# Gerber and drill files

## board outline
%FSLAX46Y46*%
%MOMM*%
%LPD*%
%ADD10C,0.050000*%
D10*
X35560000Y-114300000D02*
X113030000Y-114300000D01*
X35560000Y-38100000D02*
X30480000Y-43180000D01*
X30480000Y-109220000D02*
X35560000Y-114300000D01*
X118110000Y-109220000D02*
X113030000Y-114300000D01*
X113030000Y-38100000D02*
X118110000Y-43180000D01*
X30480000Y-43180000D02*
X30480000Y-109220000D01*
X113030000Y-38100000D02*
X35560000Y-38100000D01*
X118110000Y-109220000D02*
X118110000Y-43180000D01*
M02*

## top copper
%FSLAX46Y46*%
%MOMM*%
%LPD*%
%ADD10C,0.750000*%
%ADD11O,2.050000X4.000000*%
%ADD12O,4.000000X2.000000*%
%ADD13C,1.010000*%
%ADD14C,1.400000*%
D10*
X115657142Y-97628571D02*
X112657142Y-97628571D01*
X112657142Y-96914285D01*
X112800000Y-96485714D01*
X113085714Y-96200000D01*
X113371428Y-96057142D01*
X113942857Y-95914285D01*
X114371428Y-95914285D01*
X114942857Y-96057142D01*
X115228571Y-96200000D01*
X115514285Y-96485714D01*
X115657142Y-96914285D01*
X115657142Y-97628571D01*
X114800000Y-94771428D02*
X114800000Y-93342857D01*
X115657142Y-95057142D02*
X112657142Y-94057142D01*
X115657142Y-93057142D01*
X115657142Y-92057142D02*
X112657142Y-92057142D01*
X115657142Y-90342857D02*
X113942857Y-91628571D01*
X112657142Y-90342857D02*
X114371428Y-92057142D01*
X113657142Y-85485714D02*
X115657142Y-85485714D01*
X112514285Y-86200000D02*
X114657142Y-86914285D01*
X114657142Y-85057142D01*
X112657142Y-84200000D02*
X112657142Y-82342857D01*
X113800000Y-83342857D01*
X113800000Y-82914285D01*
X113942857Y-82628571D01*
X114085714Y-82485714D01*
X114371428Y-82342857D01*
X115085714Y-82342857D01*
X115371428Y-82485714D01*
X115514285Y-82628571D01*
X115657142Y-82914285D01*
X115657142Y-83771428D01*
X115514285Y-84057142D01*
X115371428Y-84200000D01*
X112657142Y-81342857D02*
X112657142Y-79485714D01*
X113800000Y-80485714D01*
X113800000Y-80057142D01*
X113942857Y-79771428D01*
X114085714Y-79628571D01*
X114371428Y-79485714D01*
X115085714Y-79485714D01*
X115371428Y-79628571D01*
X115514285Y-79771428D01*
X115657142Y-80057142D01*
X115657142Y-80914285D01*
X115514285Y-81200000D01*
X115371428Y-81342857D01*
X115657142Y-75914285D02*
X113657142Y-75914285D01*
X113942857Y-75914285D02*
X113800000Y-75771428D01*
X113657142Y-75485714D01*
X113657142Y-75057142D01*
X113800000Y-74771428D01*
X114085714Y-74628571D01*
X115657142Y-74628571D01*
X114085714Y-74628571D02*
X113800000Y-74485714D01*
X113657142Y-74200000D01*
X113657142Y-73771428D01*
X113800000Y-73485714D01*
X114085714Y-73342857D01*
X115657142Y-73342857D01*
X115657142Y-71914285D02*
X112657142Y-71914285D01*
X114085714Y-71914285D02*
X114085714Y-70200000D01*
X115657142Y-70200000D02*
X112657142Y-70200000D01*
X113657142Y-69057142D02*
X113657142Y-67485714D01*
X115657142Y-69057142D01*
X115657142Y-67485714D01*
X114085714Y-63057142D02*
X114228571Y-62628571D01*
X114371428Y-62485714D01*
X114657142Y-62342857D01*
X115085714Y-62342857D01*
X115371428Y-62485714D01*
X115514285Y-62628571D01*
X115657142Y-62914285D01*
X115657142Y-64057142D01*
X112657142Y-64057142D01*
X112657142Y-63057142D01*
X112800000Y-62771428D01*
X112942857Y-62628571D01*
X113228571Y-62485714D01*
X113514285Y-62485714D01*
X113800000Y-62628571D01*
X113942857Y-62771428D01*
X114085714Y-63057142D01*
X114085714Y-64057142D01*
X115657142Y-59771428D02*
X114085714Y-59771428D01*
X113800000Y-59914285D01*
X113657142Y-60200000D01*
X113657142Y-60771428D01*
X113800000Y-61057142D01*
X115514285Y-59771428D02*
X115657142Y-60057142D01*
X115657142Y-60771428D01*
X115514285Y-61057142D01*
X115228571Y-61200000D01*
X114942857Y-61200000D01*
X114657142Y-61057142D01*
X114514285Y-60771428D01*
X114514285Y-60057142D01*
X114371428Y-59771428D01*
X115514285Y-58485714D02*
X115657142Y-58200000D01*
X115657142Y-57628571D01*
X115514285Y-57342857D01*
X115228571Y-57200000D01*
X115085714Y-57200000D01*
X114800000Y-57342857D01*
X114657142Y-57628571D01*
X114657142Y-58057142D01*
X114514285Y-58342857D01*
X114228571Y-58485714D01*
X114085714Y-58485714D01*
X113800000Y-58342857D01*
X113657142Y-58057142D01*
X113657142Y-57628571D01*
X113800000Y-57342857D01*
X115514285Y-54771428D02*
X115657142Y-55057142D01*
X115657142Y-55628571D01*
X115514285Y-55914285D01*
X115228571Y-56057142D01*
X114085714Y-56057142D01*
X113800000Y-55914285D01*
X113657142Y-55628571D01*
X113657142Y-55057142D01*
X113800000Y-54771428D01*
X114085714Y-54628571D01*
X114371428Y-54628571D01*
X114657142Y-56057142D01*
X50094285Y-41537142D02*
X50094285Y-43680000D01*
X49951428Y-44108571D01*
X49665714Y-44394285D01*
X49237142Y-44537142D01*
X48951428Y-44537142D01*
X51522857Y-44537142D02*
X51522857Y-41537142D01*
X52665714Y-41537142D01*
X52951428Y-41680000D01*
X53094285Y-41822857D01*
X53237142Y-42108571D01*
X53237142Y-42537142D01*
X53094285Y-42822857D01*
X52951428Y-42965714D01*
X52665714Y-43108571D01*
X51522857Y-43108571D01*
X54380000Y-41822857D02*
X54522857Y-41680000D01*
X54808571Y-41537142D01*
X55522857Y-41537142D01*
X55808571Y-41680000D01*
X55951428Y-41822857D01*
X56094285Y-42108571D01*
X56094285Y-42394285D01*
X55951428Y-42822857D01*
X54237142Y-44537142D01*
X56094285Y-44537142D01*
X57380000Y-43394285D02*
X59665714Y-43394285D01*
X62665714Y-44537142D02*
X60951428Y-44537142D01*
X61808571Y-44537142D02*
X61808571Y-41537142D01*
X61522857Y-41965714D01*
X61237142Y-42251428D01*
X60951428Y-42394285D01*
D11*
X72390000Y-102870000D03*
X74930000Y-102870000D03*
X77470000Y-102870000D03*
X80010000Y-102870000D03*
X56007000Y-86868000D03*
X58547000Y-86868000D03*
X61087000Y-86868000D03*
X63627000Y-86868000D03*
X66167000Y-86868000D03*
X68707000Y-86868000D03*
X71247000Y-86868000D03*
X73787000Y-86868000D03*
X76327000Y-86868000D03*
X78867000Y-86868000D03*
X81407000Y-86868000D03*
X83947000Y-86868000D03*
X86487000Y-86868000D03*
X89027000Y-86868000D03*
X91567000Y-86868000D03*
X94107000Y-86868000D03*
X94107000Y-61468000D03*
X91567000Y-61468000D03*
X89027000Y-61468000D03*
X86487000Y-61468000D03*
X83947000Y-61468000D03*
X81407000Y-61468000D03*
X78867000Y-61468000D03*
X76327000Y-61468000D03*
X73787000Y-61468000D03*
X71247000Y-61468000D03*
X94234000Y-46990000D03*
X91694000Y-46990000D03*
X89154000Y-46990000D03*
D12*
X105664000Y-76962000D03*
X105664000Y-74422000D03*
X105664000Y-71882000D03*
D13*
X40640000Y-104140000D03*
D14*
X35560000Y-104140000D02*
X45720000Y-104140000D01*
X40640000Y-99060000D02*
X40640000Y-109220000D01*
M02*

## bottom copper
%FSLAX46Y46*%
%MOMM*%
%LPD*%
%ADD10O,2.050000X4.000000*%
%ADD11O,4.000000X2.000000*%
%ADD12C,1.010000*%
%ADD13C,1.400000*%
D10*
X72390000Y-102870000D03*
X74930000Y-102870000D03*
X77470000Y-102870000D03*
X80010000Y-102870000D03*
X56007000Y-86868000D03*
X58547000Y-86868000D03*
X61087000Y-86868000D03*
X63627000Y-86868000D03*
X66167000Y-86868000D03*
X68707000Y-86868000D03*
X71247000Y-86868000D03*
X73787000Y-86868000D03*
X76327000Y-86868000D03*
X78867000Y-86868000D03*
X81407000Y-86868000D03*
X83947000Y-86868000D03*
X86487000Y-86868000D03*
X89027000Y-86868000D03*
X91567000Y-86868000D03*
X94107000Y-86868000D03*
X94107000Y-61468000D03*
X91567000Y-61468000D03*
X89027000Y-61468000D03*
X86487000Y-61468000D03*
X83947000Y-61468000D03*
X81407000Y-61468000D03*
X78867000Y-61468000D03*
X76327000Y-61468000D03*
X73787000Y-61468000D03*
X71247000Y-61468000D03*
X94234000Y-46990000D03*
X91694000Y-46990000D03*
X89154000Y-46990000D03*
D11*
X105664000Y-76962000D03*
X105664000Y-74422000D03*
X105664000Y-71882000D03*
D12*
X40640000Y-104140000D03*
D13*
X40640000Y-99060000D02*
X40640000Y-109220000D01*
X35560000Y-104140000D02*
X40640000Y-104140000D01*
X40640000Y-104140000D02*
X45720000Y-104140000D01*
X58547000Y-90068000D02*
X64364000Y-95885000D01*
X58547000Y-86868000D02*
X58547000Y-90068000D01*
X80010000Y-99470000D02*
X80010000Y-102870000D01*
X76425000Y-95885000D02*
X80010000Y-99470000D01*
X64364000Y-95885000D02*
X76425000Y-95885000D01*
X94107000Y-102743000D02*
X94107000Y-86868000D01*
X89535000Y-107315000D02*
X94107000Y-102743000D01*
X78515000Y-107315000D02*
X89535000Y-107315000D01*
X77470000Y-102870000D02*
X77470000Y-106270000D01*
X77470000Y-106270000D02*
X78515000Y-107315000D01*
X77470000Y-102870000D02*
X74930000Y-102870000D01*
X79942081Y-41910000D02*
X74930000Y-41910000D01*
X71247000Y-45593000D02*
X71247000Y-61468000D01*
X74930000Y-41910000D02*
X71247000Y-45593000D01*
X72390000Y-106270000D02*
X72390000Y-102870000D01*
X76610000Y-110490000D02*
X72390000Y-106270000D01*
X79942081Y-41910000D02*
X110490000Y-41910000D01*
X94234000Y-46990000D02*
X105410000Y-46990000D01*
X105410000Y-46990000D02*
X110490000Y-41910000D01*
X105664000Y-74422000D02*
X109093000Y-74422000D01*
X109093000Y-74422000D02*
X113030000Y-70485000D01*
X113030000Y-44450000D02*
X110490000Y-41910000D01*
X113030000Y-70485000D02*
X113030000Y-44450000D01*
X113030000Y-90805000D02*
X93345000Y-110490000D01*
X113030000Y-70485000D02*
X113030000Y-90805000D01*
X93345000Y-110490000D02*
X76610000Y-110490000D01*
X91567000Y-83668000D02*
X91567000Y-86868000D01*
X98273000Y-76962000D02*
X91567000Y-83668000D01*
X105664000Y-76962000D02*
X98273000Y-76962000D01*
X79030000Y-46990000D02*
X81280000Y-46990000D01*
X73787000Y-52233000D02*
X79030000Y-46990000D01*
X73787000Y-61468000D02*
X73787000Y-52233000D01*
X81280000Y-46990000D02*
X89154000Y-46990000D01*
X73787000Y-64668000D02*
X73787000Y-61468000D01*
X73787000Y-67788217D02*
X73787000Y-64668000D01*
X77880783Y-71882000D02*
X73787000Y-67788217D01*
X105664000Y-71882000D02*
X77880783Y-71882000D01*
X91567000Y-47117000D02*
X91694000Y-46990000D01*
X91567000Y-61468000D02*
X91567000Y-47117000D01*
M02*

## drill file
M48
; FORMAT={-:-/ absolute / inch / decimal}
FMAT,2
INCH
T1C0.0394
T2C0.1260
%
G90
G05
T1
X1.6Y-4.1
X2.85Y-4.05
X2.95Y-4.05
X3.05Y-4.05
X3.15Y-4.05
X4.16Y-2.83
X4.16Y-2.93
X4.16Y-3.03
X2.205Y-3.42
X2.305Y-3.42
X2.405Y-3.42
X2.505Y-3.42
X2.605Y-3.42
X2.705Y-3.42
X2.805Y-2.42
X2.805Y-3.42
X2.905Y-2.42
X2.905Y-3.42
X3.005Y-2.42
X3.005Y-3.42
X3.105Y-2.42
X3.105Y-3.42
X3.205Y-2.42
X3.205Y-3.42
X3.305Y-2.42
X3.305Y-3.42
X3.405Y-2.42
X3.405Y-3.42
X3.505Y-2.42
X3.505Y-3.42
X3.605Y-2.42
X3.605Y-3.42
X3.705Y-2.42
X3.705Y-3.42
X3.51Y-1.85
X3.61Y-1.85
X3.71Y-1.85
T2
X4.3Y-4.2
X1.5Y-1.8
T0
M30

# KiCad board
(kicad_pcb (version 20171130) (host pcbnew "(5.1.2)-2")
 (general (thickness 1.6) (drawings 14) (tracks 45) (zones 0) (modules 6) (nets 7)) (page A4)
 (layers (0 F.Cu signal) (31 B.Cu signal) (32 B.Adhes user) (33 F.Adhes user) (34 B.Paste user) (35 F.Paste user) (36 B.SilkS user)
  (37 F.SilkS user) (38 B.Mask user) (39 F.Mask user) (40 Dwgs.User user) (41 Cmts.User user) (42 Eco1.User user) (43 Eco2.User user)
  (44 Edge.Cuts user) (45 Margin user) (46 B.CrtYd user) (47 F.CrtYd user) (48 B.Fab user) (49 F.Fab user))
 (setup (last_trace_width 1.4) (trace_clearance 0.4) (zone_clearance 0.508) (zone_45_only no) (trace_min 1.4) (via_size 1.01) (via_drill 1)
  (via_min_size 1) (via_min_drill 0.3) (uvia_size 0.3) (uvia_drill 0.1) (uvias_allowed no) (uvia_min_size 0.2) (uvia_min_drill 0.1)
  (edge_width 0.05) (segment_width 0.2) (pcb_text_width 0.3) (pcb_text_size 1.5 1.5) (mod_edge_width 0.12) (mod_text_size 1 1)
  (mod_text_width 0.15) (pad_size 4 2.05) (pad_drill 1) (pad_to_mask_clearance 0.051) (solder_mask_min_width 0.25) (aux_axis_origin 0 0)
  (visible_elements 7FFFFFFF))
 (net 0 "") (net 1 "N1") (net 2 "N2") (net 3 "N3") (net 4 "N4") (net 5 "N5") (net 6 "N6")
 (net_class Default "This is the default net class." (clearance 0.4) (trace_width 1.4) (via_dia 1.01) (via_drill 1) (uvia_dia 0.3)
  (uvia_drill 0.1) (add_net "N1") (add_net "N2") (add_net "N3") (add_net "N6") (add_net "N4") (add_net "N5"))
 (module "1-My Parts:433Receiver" (layer F.Cu) (at 72.39 102.87 90)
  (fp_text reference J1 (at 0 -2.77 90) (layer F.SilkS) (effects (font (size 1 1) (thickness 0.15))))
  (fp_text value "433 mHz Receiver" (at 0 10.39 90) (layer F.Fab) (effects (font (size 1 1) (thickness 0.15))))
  (pad 1 thru_hole oval (at 0 0 90) (size 4 2.05) (drill 1) (layers *.Cu *.Mask) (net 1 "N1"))
  (pad 2 thru_hole oval (at 0 2.54 90) (size 4 2.05) (drill 1) (layers *.Cu *.Mask) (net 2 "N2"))
  (pad 3 thru_hole oval (at 0 5.08 90) (size 4 2.05) (drill 1) (layers *.Cu *.Mask) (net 2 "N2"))
  (pad 4 thru_hole oval (at 0 7.62 90) (size 4 2.05) (drill 1) (layers *.Cu *.Mask) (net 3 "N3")))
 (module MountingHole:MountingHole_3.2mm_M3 (layer F.Cu) (at 109.22 106.68)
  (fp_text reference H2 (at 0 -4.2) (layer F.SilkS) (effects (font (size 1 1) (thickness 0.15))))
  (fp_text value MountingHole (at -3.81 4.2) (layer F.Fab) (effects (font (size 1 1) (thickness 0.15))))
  (pad 1 np_thru_hole circle (at 0 0) (size 3.2 3.2) (drill 3.2) (layers *.Cu *.Mask)))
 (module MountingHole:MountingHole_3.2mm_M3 (layer F.Cu) (at 38.1 45.72)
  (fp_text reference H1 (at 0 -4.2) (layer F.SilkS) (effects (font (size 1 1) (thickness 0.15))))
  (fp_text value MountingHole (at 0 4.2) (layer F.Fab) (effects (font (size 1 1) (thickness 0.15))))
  (pad 1 np_thru_hole circle (at 0 0) (size 3.2 3.2) (drill 3.2) (layers *.Cu *.Mask)))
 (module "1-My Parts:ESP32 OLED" (layer F.Cu) (at 31.877 60.198 270)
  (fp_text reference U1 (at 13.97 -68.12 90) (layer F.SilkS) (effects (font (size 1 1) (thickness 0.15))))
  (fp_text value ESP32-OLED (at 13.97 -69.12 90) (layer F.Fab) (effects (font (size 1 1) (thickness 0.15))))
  (pad 1 thru_hole oval (at 26.67 -24.13 270) (size 4 2.05) (drill 1) (layers *.Cu *.Mask))
  (pad 2 thru_hole oval (at 26.67 -26.67 270) (size 4 2.05) (drill 1) (layers *.Cu *.Mask) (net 3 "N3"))
  (pad 3 thru_hole oval (at 26.67 -29.21 270) (size 4 2.05) (drill 1) (layers *.Cu *.Mask))
  (pad 4 thru_hole oval (at 26.67 -31.75 270) (size 4 2.05) (drill 1) (layers *.Cu *.Mask))
  (pad 5 thru_hole oval (at 26.67 -34.29 270) (size 4 2.05) (drill 1) (layers *.Cu *.Mask))
  (pad 6 thru_hole oval (at 26.67 -36.83 270) (size 4 2.05) (drill 1) (layers *.Cu *.Mask))
  (pad 7 thru_hole oval (at 26.67 -39.37 270) (size 4 2.05) (drill 1) (layers *.Cu *.Mask))
  (pad 8 thru_hole oval (at 26.67 -41.91 270) (size 4 2.05) (drill 1) (layers *.Cu *.Mask))
  (pad 9 thru_hole oval (at 26.67 -44.45 270) (size 4 2.05) (drill 1) (layers *.Cu *.Mask))
  (pad 10 thru_hole oval (at 26.67 -46.99 270) (size 4 2.05) (drill 1) (layers *.Cu *.Mask))
  (pad 11 thru_hole oval (at 26.67 -49.53 270) (size 4 2.05) (drill 1) (layers *.Cu *.Mask))
  (pad 12 thru_hole oval (at 26.67 -52.07 270) (size 4 2.05) (drill 1) (layers *.Cu *.Mask))
  (pad 13 thru_hole oval (at 26.67 -54.61 270) (size 4 2.05) (drill 1) (layers *.Cu *.Mask))
  (pad 14 thru_hole oval (at 26.67 -57.15 270) (size 4 2.05) (drill 1) (layers *.Cu *.Mask))
  (pad 15 thru_hole oval (at 26.67 -59.69 270) (size 4 2.05) (drill 1) (layers *.Cu *.Mask) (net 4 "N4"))
  (pad 16 thru_hole oval (at 26.67 -62.23 270) (size 4 2.05) (drill 1) (layers *.Cu *.Mask) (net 2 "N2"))
  (pad 17 thru_hole oval (at 1.27 -62.23 270) (size 4 2.05) (drill 1) (layers *.Cu *.Mask))
  (pad 18 thru_hole oval (at 1.27 -59.69 270) (size 4 2.05) (drill 1) (layers *.Cu *.Mask) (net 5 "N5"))
  (pad 19 thru_hole oval (at 1.27 -57.15 270) (size 4 2.05) (drill 1) (layers *.Cu *.Mask))
  (pad 20 thru_hole oval (at 1.27 -54.61 270) (size 4 2.05) (drill 1) (layers *.Cu *.Mask))
  (pad 21 thru_hole oval (at 1.27 -52.07 270) (size 4 2.05) (drill 1) (layers *.Cu *.Mask))
  (pad 22 thru_hole oval (at 1.27 -49.53 270) (size 4 2.05) (drill 1) (layers *.Cu *.Mask))
  (pad 23 thru_hole oval (at 1.27 -46.99 270) (size 4 2.05) (drill 1) (layers *.Cu *.Mask))
  (pad 24 thru_hole oval (at 1.27 -44.45 270) (size 4 2.05) (drill 1) (layers *.Cu *.Mask))
  (pad 25 thru_hole oval (at 1.27 -41.91 270) (size 4 2.05) (drill 1) (layers *.Cu *.Mask) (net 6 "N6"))
  (pad 26 thru_hole oval (at 1.27 -39.37 270) (size 4 2.05) (drill 1) (layers *.Cu *.Mask) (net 1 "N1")))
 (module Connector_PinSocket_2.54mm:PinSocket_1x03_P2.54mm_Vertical (layer F.Cu) (at 89.154 46.99 90)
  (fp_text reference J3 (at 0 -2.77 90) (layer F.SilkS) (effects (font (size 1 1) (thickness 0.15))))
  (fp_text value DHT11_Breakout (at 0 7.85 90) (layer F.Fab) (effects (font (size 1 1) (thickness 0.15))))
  (pad 3 thru_hole oval (at 0 5.08 90) (size 4 2.05) (drill 1) (layers *.Cu *.Mask) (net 1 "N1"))
  (pad 2 thru_hole oval (at 0 2.54 90) (size 4 2.05) (drill 1) (layers *.Cu *.Mask) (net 5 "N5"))
  (pad 1 thru_hole oval (at 0 0 90) (size 4 2.05) (drill 1) (layers *.Cu *.Mask) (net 6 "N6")))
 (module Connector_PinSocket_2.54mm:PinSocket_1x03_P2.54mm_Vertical (layer F.Cu) (at 105.664 71.882)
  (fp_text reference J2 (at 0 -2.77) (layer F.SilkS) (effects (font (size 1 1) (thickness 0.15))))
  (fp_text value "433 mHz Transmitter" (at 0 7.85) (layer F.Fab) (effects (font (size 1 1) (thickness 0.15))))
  (pad 3 thru_hole oval (at 0 5.08) (size 4 2) (drill 1) (layers *.Cu *.Mask) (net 4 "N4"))
  (pad 2 thru_hole oval (at 0 2.54) (size 4 2) (drill 1) (layers *.Cu *.Mask) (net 1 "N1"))
  (pad 1 thru_hole oval (at 0 0) (size 4 2) (drill 1) (layers *.Cu *.Mask) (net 6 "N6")))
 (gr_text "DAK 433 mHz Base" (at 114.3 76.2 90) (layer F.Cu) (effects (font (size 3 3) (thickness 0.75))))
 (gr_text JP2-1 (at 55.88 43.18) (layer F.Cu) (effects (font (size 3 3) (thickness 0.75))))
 (gr_line (start 35.56 114.3) (end 113.03 114.3) (layer Edge.Cuts) (width 0.05))
 (gr_line (start 35.56 38.1) (end 30.48 43.18) (layer Edge.Cuts) (width 0.05))
 (gr_line (start 30.48 109.22) (end 35.56 114.3) (layer Edge.Cuts) (width 0.05))
 (gr_line (start 118.11 109.22) (end 113.03 114.3) (layer Edge.Cuts) (width 0.05))
 (gr_line (start 113.03 38.1) (end 118.11 43.18) (layer Edge.Cuts) (width 0.05))
 (gr_line (start 30.48 43.18) (end 30.48 109.22) (layer Edge.Cuts) (width 0.05))
 (gr_line (start 113.03 38.1) (end 35.56 38.1) (layer Edge.Cuts) (width 0.05))
 (gr_line (start 118.11 109.22) (end 118.11 43.18) (layer Edge.Cuts) (width 0.05))
 (segment (start 40.64 99.06) (end 40.64 109.22) (width 1.4) (layer B.Cu) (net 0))
 (segment (start 35.56 104.14) (end 45.72 104.14) (width 1.4) (layer F.Cu) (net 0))
 (segment (start 35.56 104.14) (end 40.64 104.14) (width 1.4) (layer B.Cu) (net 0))
 (segment (start 40.64 99.06) (end 40.64 109.22) (width 1.4) (layer F.Cu) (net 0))
 (segment (start 40.64 104.14) (end 45.72 104.14) (width 1.4) (layer B.Cu) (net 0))
 (via (at 40.64 104.14) (size 1.01) (drill 1) (layers F.Cu B.Cu) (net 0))
 (segment (start 58.547 90.068) (end 64.364 95.885) (width 1.4) (layer B.Cu) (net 3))
 (segment (start 58.547 86.868) (end 58.547 90.068) (width 1.4) (layer B.Cu) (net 3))
 (segment (start 80.01 99.47) (end 80.01 102.87) (width 1.4) (layer B.Cu) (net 3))
 (segment (start 76.425 95.885) (end 80.01 99.47) (width 1.4) (layer B.Cu) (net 3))
 (segment (start 64.364 95.885) (end 76.425 95.885) (width 1.4) (layer B.Cu) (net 3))
 (segment (start 94.107 102.743) (end 94.107 86.868) (width 1.4) (layer B.Cu) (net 2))
 (segment (start 89.535 107.315) (end 94.107 102.743) (width 1.4) (layer B.Cu) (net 2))
 (segment (start 78.515 107.315) (end 89.535 107.315) (width 1.4) (layer B.Cu) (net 2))
 (segment (start 77.47 102.87) (end 77.47 106.27) (width 1.4) (layer B.Cu) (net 2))
 (segment (start 77.47 106.27) (end 78.515 107.315) (width 1.4) (layer B.Cu) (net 2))
 (segment (start 77.47 102.87) (end 74.93 102.87) (width 1.4) (layer B.Cu) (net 2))
 (segment (start 79.942081 41.91) (end 74.93 41.91) (width 1.4) (layer B.Cu) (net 1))
 (segment (start 71.247 45.593) (end 71.247 61.468) (width 1.4) (layer B.Cu) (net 1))
 (segment (start 74.93 41.91) (end 71.247 45.593) (width 1.4) (layer B.Cu) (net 1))
 (segment (start 72.39 106.27) (end 72.39 102.87) (width 1.4) (layer B.Cu) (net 1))
 (segment (start 76.61 110.49) (end 72.39 106.27) (width 1.4) (layer B.Cu) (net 1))
 (segment (start 79.942081 41.91) (end 110.49 41.91) (width 1.4) (layer B.Cu) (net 1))
 (segment (start 94.234 46.99) (end 105.41 46.99) (width 1.4) (layer B.Cu) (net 1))
 (segment (start 105.41 46.99) (end 110.49 41.91) (width 1.4) (layer B.Cu) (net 1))
 (segment (start 105.664 74.422) (end 109.093 74.422) (width 1.4) (layer B.Cu) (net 1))
 (segment (start 109.093 74.422) (end 113.03 70.485) (width 1.4) (layer B.Cu) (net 1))
 (segment (start 113.03 44.45) (end 110.49 41.91) (width 1.4) (layer B.Cu) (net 1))
 (segment (start 113.03 70.485) (end 113.03 44.45) (width 1.4) (layer B.Cu) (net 1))
 (segment (start 113.03 90.805) (end 93.345 110.49) (width 1.4) (layer B.Cu) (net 1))
 (segment (start 113.03 70.485) (end 113.03 90.805) (width 1.4) (layer B.Cu) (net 1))
 (segment (start 93.345 110.49) (end 76.61 110.49) (width 1.4) (layer B.Cu) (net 1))
 (segment (start 91.567 83.668) (end 91.567 86.868) (width 1.4) (layer B.Cu) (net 4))
 (segment (start 98.273 76.962) (end 91.567 83.668) (width 1.4) (layer B.Cu) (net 4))
 (segment (start 105.664 76.962) (end 98.273 76.962) (width 1.4) (layer B.Cu) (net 4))
 (segment (start 79.03 46.99) (end 81.28 46.99) (width 1.4) (layer B.Cu) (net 6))
 (segment (start 73.787 52.233) (end 79.03 46.99) (width 1.4) (layer B.Cu) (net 6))
 (segment (start 73.787 61.468) (end 73.787 52.233) (width 1.4) (layer B.Cu) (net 6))
 (segment (start 81.28 46.99) (end 89.154 46.99) (width 1.4) (layer B.Cu) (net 6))
 (segment (start 73.787 64.668) (end 73.787 61.468) (width 1.4) (layer B.Cu) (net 6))
 (segment (start 73.787 67.788217) (end 73.787 64.668) (width 1.4) (layer B.Cu) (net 6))
 (segment (start 77.880783 71.882) (end 73.787 67.788217) (width 1.4) (layer B.Cu) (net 6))
 (segment (start 105.664 71.882) (end 77.880783 71.882) (width 1.4) (layer B.Cu) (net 6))
 (segment (start 91.567 47.117) (end 91.694 46.99) (width 1.4) (layer B.Cu) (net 5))
 (segment (start 91.567 61.468) (end 91.567 47.117) (width 1.4) (layer B.Cu) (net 5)))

